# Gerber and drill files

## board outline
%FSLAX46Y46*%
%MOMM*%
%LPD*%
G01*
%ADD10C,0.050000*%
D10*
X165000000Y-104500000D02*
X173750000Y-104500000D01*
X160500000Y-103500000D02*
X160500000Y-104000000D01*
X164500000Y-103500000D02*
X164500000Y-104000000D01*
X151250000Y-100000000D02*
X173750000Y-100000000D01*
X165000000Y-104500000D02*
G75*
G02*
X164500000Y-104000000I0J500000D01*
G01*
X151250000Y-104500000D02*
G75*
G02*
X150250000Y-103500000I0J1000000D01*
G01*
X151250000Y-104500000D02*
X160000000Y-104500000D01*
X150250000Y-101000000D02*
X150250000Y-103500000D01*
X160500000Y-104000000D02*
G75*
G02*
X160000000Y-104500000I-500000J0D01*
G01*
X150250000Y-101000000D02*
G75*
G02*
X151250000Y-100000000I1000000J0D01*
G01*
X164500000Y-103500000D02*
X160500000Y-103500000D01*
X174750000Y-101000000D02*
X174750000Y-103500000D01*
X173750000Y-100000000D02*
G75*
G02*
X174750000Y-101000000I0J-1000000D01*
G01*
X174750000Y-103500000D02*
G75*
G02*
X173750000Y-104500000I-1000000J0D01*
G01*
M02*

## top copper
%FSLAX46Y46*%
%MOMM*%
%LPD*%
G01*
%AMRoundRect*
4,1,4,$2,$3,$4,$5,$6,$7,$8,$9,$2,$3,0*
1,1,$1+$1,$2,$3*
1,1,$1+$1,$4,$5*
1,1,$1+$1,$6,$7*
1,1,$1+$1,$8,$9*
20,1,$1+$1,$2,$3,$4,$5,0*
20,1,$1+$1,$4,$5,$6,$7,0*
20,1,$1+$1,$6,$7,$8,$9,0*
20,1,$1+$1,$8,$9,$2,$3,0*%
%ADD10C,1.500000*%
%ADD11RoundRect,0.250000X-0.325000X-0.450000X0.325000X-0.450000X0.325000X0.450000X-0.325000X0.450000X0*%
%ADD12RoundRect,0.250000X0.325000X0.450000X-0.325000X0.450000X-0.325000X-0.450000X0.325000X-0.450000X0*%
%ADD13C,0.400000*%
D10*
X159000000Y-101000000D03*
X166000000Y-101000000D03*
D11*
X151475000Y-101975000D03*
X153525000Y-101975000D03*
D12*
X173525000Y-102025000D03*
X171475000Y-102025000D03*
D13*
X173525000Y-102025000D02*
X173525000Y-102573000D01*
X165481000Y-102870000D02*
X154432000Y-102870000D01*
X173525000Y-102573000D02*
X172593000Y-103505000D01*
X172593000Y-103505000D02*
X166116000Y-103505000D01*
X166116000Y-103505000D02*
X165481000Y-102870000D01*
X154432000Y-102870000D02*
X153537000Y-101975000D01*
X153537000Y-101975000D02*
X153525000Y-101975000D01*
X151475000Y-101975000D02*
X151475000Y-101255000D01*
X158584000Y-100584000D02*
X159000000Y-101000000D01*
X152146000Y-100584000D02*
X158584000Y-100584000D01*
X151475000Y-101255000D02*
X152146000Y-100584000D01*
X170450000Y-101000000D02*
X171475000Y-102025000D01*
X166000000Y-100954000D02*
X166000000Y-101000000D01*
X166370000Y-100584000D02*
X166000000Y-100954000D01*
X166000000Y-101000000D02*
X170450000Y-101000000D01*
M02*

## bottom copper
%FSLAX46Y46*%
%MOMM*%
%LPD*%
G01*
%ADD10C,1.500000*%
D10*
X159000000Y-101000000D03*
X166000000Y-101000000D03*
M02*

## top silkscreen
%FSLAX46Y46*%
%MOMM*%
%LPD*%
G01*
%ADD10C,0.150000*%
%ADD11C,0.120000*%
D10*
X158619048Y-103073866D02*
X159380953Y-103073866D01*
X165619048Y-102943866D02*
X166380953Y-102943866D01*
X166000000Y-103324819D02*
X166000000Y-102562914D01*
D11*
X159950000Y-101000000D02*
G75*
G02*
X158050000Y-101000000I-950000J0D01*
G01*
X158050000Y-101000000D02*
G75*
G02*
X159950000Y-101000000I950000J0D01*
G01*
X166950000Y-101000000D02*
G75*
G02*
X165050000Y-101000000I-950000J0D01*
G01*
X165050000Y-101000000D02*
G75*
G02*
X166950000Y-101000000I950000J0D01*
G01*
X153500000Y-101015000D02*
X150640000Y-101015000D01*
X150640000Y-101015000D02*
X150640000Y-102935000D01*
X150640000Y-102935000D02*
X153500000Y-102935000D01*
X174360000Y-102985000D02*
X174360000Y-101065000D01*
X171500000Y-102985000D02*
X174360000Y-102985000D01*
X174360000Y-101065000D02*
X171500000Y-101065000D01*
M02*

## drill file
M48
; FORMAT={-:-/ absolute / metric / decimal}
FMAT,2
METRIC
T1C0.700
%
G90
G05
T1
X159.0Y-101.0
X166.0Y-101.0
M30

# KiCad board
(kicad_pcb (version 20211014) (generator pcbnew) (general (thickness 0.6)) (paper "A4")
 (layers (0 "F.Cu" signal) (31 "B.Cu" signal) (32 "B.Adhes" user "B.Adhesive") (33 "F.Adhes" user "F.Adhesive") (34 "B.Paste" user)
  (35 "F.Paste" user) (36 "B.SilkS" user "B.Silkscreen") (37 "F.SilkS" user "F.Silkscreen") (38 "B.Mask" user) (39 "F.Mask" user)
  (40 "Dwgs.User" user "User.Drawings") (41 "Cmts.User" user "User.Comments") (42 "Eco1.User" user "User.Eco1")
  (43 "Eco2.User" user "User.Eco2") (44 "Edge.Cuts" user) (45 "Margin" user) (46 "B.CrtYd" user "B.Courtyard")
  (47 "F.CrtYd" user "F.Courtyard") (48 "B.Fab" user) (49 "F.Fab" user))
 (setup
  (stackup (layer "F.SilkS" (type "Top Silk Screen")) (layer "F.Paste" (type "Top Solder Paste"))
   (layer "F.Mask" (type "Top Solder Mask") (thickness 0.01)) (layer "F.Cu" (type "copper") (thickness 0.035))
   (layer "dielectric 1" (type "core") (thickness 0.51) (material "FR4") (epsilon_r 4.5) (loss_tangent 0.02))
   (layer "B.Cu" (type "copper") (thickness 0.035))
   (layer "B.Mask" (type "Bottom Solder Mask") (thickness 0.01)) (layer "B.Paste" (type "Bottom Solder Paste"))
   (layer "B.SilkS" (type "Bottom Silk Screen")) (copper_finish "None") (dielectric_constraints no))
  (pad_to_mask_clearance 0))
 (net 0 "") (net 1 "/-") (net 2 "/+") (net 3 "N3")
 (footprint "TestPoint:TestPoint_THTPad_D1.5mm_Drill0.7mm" (layer "F.Cu") (at 159 101)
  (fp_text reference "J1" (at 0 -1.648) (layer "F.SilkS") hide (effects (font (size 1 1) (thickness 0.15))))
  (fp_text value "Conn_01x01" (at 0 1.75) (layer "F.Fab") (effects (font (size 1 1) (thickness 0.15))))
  (fp_circle (center 0 0) (end 0 0.95) (layer "F.SilkS") (width 0.12) (fill none))
  (pad "1" thru_hole circle locked (at 0 0) (size 1.5 1.5) (drill 0.7) (layers *.Cu *.Mask) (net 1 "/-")))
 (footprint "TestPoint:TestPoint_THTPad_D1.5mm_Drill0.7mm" (layer "F.Cu") (at 166 101)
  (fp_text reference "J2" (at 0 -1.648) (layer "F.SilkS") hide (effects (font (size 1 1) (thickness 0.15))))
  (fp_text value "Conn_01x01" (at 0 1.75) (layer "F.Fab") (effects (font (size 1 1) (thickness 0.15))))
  (fp_circle (center 0 0) (end 0 0.95) (layer "F.SilkS") (width 0.12) (fill none))
  (pad "1" thru_hole circle locked (at 0 0) (size 1.5 1.5) (drill 0.7) (layers *.Cu *.Mask) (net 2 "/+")))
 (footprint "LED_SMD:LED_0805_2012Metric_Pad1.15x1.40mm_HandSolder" (layer "F.Cu") (at 152.5 101.975)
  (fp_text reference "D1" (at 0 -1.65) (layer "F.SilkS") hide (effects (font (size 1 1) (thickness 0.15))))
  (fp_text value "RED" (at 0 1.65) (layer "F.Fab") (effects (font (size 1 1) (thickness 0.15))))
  (fp_line (start 1 -0.96) (end -1.86 -0.96) (layer "F.SilkS") (width 0.12))
  (fp_line (start -1.86 -0.96) (end -1.86 0.96) (layer "F.SilkS") (width 0.12))
  (fp_line (start -1.86 0.96) (end 1 0.96) (layer "F.SilkS") (width 0.12))
  (pad "1" smd roundrect locked (at -1.025 0) (size 1.15 1.4) (layers "F.Cu" "F.Paste" "F.Mask") (roundrect_rratio 0.217391) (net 1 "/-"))
  (pad "2" smd roundrect locked (at 1.025 0) (size 1.15 1.4) (layers "F.Cu" "F.Paste" "F.Mask") (roundrect_rratio 0.217391) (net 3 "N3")))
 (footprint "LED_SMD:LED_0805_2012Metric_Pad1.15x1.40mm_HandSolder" (layer "F.Cu") (at 172.5 102.025 180)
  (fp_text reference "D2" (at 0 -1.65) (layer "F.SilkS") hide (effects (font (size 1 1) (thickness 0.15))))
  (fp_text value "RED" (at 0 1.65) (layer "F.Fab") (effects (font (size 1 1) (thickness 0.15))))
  (fp_line (start -1.86 -0.96) (end -1.86 0.96) (layer "F.SilkS") (width 0.12))
  (fp_line (start 1 -0.96) (end -1.86 -0.96) (layer "F.SilkS") (width 0.12))
  (fp_line (start -1.86 0.96) (end 1 0.96) (layer "F.SilkS") (width 0.12))
  (pad "1" smd roundrect locked (at -1.025 0 180) (size 1.15 1.4) (layers "F.Cu" "F.Paste" "F.Mask") (roundrect_rratio 0.217391)
   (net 3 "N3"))
  (pad "2" smd roundrect locked (at 1.025 0 180) (size 1.15 1.4) (layers "F.Cu" "F.Paste" "F.Mask") (roundrect_rratio 0.217391) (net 2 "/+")))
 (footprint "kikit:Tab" (layer "F.Cu") (at 175 102.25 180)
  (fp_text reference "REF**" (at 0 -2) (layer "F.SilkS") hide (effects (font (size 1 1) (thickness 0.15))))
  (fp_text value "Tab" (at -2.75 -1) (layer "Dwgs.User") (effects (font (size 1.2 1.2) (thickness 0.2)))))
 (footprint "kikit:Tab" (layer "F.Cu") (at 154.5 99.75 -90)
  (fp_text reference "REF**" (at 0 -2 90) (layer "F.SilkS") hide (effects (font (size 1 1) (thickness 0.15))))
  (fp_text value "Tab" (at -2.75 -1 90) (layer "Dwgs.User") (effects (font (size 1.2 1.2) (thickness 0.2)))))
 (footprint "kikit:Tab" (layer "F.Cu") (at 170.25 104.75 90)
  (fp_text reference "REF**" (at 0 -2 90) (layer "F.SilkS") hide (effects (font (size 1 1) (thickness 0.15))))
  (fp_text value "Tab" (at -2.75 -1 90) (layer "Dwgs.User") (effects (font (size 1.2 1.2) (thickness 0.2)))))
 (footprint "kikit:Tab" (layer "F.Cu") (at 170.25 99.75 -90)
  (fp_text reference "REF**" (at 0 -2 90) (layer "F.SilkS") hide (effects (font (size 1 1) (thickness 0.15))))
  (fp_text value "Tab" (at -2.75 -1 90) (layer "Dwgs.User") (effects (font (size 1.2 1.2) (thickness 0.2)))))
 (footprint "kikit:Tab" (layer "F.Cu") (at 154.5 104.75 90)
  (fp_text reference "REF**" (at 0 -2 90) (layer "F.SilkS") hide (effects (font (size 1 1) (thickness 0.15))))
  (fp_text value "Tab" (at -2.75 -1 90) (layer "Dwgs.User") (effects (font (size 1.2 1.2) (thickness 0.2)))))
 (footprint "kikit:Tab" (layer "F.Cu") (at 150 102.25)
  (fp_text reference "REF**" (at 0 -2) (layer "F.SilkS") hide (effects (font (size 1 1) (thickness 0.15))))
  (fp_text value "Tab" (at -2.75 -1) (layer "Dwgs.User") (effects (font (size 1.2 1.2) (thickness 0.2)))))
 (gr_line (start 165 104.5) (end 173.75 104.5) (layer "Edge.Cuts") (width 0.05))
 (gr_line (start 160.5 103.5) (end 160.5 104) (layer "Edge.Cuts") (width 0.05))
 (gr_line (start 164.5 103.5) (end 164.5 104) (layer "Edge.Cuts") (width 0.05))
 (gr_line (start 151.25 100) (end 173.75 100) (layer "Edge.Cuts") (width 0.05))
 (gr_arc (start 165 104.5) (mid 164.646447 104.353553) (end 164.5 104) (layer "Edge.Cuts") (width 0.05))
 (gr_arc (start 151.25 104.5) (mid 150.542893 104.207107) (end 150.25 103.5) (layer "Edge.Cuts") (width 0.05))
 (gr_line (start 151.25 104.5) (end 160 104.5) (layer "Edge.Cuts") (width 0.05))
 (gr_line (start 150.25 101) (end 150.25 103.5) (layer "Edge.Cuts") (width 0.05))
 (gr_arc (start 160.5 104) (mid 160.353553 104.353553) (end 160 104.5) (layer "Edge.Cuts") (width 0.05))
 (gr_arc (start 150.25 101) (mid 150.542893 100.292893) (end 151.25 100) (layer "Edge.Cuts") (width 0.05))
 (gr_line (start 164.5 103.5) (end 160.5 103.5) (layer "Edge.Cuts") (width 0.05))
 (gr_line (start 174.75 101) (end 174.75 103.5) (layer "Edge.Cuts") (width 0.05))
 (gr_arc (start 173.75 100) (mid 174.457107 100.292893) (end 174.75 101) (layer "Edge.Cuts") (width 0.05))
 (gr_arc (start 174.75 103.5) (mid 174.457107 104.207107) (end 173.75 104.5) (layer "Edge.Cuts") (width 0.05))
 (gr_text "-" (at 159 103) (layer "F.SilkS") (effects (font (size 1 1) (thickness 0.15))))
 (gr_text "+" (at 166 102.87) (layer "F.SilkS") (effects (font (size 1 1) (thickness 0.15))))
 (segment (start 173.525 102.025) (end 173.525 102.573) (width 0.4) (layer "F.Cu") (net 3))
 (segment (start 165.481 102.87) (end 154.432 102.87) (width 0.4) (layer "F.Cu") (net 3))
 (segment (start 173.525 102.573) (end 172.593 103.505) (width 0.4) (layer "F.Cu") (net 3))
 (segment (start 172.593 103.505) (end 166.116 103.505) (width 0.4) (layer "F.Cu") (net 3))
 (segment (start 166.116 103.505) (end 165.481 102.87) (width 0.4) (layer "F.Cu") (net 3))
 (segment (start 154.432 102.87) (end 153.537 101.975) (width 0.4) (layer "F.Cu") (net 3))
 (segment (start 153.537 101.975) (end 153.525 101.975) (width 0.4) (layer "F.Cu") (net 3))
 (segment (start 151.475 101.975) (end 151.475 101.255) (width 0.4) (layer "F.Cu") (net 1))
 (segment (start 158.584 100.584) (end 159 101) (width 0.4) (layer "F.Cu") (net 1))
 (segment (start 152.146 100.584) (end 158.584 100.584) (width 0.4) (layer "F.Cu") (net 1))
 (segment (start 151.475 101.255) (end 152.146 100.584) (width 0.4) (layer "F.Cu") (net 1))
 (segment (start 170.45 101) (end 171.475 102.025) (width 0.4) (layer "F.Cu") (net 2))
 (segment (start 166 100.954) (end 166 101) (width 0.4) (layer "F.Cu") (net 2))
 (segment (start 166.37 100.584) (end 166 100.954) (width 0.4) (layer "F.Cu") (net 2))
 (segment (start 166 101) (end 170.45 101) (width 0.4) (layer "F.Cu") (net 2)))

